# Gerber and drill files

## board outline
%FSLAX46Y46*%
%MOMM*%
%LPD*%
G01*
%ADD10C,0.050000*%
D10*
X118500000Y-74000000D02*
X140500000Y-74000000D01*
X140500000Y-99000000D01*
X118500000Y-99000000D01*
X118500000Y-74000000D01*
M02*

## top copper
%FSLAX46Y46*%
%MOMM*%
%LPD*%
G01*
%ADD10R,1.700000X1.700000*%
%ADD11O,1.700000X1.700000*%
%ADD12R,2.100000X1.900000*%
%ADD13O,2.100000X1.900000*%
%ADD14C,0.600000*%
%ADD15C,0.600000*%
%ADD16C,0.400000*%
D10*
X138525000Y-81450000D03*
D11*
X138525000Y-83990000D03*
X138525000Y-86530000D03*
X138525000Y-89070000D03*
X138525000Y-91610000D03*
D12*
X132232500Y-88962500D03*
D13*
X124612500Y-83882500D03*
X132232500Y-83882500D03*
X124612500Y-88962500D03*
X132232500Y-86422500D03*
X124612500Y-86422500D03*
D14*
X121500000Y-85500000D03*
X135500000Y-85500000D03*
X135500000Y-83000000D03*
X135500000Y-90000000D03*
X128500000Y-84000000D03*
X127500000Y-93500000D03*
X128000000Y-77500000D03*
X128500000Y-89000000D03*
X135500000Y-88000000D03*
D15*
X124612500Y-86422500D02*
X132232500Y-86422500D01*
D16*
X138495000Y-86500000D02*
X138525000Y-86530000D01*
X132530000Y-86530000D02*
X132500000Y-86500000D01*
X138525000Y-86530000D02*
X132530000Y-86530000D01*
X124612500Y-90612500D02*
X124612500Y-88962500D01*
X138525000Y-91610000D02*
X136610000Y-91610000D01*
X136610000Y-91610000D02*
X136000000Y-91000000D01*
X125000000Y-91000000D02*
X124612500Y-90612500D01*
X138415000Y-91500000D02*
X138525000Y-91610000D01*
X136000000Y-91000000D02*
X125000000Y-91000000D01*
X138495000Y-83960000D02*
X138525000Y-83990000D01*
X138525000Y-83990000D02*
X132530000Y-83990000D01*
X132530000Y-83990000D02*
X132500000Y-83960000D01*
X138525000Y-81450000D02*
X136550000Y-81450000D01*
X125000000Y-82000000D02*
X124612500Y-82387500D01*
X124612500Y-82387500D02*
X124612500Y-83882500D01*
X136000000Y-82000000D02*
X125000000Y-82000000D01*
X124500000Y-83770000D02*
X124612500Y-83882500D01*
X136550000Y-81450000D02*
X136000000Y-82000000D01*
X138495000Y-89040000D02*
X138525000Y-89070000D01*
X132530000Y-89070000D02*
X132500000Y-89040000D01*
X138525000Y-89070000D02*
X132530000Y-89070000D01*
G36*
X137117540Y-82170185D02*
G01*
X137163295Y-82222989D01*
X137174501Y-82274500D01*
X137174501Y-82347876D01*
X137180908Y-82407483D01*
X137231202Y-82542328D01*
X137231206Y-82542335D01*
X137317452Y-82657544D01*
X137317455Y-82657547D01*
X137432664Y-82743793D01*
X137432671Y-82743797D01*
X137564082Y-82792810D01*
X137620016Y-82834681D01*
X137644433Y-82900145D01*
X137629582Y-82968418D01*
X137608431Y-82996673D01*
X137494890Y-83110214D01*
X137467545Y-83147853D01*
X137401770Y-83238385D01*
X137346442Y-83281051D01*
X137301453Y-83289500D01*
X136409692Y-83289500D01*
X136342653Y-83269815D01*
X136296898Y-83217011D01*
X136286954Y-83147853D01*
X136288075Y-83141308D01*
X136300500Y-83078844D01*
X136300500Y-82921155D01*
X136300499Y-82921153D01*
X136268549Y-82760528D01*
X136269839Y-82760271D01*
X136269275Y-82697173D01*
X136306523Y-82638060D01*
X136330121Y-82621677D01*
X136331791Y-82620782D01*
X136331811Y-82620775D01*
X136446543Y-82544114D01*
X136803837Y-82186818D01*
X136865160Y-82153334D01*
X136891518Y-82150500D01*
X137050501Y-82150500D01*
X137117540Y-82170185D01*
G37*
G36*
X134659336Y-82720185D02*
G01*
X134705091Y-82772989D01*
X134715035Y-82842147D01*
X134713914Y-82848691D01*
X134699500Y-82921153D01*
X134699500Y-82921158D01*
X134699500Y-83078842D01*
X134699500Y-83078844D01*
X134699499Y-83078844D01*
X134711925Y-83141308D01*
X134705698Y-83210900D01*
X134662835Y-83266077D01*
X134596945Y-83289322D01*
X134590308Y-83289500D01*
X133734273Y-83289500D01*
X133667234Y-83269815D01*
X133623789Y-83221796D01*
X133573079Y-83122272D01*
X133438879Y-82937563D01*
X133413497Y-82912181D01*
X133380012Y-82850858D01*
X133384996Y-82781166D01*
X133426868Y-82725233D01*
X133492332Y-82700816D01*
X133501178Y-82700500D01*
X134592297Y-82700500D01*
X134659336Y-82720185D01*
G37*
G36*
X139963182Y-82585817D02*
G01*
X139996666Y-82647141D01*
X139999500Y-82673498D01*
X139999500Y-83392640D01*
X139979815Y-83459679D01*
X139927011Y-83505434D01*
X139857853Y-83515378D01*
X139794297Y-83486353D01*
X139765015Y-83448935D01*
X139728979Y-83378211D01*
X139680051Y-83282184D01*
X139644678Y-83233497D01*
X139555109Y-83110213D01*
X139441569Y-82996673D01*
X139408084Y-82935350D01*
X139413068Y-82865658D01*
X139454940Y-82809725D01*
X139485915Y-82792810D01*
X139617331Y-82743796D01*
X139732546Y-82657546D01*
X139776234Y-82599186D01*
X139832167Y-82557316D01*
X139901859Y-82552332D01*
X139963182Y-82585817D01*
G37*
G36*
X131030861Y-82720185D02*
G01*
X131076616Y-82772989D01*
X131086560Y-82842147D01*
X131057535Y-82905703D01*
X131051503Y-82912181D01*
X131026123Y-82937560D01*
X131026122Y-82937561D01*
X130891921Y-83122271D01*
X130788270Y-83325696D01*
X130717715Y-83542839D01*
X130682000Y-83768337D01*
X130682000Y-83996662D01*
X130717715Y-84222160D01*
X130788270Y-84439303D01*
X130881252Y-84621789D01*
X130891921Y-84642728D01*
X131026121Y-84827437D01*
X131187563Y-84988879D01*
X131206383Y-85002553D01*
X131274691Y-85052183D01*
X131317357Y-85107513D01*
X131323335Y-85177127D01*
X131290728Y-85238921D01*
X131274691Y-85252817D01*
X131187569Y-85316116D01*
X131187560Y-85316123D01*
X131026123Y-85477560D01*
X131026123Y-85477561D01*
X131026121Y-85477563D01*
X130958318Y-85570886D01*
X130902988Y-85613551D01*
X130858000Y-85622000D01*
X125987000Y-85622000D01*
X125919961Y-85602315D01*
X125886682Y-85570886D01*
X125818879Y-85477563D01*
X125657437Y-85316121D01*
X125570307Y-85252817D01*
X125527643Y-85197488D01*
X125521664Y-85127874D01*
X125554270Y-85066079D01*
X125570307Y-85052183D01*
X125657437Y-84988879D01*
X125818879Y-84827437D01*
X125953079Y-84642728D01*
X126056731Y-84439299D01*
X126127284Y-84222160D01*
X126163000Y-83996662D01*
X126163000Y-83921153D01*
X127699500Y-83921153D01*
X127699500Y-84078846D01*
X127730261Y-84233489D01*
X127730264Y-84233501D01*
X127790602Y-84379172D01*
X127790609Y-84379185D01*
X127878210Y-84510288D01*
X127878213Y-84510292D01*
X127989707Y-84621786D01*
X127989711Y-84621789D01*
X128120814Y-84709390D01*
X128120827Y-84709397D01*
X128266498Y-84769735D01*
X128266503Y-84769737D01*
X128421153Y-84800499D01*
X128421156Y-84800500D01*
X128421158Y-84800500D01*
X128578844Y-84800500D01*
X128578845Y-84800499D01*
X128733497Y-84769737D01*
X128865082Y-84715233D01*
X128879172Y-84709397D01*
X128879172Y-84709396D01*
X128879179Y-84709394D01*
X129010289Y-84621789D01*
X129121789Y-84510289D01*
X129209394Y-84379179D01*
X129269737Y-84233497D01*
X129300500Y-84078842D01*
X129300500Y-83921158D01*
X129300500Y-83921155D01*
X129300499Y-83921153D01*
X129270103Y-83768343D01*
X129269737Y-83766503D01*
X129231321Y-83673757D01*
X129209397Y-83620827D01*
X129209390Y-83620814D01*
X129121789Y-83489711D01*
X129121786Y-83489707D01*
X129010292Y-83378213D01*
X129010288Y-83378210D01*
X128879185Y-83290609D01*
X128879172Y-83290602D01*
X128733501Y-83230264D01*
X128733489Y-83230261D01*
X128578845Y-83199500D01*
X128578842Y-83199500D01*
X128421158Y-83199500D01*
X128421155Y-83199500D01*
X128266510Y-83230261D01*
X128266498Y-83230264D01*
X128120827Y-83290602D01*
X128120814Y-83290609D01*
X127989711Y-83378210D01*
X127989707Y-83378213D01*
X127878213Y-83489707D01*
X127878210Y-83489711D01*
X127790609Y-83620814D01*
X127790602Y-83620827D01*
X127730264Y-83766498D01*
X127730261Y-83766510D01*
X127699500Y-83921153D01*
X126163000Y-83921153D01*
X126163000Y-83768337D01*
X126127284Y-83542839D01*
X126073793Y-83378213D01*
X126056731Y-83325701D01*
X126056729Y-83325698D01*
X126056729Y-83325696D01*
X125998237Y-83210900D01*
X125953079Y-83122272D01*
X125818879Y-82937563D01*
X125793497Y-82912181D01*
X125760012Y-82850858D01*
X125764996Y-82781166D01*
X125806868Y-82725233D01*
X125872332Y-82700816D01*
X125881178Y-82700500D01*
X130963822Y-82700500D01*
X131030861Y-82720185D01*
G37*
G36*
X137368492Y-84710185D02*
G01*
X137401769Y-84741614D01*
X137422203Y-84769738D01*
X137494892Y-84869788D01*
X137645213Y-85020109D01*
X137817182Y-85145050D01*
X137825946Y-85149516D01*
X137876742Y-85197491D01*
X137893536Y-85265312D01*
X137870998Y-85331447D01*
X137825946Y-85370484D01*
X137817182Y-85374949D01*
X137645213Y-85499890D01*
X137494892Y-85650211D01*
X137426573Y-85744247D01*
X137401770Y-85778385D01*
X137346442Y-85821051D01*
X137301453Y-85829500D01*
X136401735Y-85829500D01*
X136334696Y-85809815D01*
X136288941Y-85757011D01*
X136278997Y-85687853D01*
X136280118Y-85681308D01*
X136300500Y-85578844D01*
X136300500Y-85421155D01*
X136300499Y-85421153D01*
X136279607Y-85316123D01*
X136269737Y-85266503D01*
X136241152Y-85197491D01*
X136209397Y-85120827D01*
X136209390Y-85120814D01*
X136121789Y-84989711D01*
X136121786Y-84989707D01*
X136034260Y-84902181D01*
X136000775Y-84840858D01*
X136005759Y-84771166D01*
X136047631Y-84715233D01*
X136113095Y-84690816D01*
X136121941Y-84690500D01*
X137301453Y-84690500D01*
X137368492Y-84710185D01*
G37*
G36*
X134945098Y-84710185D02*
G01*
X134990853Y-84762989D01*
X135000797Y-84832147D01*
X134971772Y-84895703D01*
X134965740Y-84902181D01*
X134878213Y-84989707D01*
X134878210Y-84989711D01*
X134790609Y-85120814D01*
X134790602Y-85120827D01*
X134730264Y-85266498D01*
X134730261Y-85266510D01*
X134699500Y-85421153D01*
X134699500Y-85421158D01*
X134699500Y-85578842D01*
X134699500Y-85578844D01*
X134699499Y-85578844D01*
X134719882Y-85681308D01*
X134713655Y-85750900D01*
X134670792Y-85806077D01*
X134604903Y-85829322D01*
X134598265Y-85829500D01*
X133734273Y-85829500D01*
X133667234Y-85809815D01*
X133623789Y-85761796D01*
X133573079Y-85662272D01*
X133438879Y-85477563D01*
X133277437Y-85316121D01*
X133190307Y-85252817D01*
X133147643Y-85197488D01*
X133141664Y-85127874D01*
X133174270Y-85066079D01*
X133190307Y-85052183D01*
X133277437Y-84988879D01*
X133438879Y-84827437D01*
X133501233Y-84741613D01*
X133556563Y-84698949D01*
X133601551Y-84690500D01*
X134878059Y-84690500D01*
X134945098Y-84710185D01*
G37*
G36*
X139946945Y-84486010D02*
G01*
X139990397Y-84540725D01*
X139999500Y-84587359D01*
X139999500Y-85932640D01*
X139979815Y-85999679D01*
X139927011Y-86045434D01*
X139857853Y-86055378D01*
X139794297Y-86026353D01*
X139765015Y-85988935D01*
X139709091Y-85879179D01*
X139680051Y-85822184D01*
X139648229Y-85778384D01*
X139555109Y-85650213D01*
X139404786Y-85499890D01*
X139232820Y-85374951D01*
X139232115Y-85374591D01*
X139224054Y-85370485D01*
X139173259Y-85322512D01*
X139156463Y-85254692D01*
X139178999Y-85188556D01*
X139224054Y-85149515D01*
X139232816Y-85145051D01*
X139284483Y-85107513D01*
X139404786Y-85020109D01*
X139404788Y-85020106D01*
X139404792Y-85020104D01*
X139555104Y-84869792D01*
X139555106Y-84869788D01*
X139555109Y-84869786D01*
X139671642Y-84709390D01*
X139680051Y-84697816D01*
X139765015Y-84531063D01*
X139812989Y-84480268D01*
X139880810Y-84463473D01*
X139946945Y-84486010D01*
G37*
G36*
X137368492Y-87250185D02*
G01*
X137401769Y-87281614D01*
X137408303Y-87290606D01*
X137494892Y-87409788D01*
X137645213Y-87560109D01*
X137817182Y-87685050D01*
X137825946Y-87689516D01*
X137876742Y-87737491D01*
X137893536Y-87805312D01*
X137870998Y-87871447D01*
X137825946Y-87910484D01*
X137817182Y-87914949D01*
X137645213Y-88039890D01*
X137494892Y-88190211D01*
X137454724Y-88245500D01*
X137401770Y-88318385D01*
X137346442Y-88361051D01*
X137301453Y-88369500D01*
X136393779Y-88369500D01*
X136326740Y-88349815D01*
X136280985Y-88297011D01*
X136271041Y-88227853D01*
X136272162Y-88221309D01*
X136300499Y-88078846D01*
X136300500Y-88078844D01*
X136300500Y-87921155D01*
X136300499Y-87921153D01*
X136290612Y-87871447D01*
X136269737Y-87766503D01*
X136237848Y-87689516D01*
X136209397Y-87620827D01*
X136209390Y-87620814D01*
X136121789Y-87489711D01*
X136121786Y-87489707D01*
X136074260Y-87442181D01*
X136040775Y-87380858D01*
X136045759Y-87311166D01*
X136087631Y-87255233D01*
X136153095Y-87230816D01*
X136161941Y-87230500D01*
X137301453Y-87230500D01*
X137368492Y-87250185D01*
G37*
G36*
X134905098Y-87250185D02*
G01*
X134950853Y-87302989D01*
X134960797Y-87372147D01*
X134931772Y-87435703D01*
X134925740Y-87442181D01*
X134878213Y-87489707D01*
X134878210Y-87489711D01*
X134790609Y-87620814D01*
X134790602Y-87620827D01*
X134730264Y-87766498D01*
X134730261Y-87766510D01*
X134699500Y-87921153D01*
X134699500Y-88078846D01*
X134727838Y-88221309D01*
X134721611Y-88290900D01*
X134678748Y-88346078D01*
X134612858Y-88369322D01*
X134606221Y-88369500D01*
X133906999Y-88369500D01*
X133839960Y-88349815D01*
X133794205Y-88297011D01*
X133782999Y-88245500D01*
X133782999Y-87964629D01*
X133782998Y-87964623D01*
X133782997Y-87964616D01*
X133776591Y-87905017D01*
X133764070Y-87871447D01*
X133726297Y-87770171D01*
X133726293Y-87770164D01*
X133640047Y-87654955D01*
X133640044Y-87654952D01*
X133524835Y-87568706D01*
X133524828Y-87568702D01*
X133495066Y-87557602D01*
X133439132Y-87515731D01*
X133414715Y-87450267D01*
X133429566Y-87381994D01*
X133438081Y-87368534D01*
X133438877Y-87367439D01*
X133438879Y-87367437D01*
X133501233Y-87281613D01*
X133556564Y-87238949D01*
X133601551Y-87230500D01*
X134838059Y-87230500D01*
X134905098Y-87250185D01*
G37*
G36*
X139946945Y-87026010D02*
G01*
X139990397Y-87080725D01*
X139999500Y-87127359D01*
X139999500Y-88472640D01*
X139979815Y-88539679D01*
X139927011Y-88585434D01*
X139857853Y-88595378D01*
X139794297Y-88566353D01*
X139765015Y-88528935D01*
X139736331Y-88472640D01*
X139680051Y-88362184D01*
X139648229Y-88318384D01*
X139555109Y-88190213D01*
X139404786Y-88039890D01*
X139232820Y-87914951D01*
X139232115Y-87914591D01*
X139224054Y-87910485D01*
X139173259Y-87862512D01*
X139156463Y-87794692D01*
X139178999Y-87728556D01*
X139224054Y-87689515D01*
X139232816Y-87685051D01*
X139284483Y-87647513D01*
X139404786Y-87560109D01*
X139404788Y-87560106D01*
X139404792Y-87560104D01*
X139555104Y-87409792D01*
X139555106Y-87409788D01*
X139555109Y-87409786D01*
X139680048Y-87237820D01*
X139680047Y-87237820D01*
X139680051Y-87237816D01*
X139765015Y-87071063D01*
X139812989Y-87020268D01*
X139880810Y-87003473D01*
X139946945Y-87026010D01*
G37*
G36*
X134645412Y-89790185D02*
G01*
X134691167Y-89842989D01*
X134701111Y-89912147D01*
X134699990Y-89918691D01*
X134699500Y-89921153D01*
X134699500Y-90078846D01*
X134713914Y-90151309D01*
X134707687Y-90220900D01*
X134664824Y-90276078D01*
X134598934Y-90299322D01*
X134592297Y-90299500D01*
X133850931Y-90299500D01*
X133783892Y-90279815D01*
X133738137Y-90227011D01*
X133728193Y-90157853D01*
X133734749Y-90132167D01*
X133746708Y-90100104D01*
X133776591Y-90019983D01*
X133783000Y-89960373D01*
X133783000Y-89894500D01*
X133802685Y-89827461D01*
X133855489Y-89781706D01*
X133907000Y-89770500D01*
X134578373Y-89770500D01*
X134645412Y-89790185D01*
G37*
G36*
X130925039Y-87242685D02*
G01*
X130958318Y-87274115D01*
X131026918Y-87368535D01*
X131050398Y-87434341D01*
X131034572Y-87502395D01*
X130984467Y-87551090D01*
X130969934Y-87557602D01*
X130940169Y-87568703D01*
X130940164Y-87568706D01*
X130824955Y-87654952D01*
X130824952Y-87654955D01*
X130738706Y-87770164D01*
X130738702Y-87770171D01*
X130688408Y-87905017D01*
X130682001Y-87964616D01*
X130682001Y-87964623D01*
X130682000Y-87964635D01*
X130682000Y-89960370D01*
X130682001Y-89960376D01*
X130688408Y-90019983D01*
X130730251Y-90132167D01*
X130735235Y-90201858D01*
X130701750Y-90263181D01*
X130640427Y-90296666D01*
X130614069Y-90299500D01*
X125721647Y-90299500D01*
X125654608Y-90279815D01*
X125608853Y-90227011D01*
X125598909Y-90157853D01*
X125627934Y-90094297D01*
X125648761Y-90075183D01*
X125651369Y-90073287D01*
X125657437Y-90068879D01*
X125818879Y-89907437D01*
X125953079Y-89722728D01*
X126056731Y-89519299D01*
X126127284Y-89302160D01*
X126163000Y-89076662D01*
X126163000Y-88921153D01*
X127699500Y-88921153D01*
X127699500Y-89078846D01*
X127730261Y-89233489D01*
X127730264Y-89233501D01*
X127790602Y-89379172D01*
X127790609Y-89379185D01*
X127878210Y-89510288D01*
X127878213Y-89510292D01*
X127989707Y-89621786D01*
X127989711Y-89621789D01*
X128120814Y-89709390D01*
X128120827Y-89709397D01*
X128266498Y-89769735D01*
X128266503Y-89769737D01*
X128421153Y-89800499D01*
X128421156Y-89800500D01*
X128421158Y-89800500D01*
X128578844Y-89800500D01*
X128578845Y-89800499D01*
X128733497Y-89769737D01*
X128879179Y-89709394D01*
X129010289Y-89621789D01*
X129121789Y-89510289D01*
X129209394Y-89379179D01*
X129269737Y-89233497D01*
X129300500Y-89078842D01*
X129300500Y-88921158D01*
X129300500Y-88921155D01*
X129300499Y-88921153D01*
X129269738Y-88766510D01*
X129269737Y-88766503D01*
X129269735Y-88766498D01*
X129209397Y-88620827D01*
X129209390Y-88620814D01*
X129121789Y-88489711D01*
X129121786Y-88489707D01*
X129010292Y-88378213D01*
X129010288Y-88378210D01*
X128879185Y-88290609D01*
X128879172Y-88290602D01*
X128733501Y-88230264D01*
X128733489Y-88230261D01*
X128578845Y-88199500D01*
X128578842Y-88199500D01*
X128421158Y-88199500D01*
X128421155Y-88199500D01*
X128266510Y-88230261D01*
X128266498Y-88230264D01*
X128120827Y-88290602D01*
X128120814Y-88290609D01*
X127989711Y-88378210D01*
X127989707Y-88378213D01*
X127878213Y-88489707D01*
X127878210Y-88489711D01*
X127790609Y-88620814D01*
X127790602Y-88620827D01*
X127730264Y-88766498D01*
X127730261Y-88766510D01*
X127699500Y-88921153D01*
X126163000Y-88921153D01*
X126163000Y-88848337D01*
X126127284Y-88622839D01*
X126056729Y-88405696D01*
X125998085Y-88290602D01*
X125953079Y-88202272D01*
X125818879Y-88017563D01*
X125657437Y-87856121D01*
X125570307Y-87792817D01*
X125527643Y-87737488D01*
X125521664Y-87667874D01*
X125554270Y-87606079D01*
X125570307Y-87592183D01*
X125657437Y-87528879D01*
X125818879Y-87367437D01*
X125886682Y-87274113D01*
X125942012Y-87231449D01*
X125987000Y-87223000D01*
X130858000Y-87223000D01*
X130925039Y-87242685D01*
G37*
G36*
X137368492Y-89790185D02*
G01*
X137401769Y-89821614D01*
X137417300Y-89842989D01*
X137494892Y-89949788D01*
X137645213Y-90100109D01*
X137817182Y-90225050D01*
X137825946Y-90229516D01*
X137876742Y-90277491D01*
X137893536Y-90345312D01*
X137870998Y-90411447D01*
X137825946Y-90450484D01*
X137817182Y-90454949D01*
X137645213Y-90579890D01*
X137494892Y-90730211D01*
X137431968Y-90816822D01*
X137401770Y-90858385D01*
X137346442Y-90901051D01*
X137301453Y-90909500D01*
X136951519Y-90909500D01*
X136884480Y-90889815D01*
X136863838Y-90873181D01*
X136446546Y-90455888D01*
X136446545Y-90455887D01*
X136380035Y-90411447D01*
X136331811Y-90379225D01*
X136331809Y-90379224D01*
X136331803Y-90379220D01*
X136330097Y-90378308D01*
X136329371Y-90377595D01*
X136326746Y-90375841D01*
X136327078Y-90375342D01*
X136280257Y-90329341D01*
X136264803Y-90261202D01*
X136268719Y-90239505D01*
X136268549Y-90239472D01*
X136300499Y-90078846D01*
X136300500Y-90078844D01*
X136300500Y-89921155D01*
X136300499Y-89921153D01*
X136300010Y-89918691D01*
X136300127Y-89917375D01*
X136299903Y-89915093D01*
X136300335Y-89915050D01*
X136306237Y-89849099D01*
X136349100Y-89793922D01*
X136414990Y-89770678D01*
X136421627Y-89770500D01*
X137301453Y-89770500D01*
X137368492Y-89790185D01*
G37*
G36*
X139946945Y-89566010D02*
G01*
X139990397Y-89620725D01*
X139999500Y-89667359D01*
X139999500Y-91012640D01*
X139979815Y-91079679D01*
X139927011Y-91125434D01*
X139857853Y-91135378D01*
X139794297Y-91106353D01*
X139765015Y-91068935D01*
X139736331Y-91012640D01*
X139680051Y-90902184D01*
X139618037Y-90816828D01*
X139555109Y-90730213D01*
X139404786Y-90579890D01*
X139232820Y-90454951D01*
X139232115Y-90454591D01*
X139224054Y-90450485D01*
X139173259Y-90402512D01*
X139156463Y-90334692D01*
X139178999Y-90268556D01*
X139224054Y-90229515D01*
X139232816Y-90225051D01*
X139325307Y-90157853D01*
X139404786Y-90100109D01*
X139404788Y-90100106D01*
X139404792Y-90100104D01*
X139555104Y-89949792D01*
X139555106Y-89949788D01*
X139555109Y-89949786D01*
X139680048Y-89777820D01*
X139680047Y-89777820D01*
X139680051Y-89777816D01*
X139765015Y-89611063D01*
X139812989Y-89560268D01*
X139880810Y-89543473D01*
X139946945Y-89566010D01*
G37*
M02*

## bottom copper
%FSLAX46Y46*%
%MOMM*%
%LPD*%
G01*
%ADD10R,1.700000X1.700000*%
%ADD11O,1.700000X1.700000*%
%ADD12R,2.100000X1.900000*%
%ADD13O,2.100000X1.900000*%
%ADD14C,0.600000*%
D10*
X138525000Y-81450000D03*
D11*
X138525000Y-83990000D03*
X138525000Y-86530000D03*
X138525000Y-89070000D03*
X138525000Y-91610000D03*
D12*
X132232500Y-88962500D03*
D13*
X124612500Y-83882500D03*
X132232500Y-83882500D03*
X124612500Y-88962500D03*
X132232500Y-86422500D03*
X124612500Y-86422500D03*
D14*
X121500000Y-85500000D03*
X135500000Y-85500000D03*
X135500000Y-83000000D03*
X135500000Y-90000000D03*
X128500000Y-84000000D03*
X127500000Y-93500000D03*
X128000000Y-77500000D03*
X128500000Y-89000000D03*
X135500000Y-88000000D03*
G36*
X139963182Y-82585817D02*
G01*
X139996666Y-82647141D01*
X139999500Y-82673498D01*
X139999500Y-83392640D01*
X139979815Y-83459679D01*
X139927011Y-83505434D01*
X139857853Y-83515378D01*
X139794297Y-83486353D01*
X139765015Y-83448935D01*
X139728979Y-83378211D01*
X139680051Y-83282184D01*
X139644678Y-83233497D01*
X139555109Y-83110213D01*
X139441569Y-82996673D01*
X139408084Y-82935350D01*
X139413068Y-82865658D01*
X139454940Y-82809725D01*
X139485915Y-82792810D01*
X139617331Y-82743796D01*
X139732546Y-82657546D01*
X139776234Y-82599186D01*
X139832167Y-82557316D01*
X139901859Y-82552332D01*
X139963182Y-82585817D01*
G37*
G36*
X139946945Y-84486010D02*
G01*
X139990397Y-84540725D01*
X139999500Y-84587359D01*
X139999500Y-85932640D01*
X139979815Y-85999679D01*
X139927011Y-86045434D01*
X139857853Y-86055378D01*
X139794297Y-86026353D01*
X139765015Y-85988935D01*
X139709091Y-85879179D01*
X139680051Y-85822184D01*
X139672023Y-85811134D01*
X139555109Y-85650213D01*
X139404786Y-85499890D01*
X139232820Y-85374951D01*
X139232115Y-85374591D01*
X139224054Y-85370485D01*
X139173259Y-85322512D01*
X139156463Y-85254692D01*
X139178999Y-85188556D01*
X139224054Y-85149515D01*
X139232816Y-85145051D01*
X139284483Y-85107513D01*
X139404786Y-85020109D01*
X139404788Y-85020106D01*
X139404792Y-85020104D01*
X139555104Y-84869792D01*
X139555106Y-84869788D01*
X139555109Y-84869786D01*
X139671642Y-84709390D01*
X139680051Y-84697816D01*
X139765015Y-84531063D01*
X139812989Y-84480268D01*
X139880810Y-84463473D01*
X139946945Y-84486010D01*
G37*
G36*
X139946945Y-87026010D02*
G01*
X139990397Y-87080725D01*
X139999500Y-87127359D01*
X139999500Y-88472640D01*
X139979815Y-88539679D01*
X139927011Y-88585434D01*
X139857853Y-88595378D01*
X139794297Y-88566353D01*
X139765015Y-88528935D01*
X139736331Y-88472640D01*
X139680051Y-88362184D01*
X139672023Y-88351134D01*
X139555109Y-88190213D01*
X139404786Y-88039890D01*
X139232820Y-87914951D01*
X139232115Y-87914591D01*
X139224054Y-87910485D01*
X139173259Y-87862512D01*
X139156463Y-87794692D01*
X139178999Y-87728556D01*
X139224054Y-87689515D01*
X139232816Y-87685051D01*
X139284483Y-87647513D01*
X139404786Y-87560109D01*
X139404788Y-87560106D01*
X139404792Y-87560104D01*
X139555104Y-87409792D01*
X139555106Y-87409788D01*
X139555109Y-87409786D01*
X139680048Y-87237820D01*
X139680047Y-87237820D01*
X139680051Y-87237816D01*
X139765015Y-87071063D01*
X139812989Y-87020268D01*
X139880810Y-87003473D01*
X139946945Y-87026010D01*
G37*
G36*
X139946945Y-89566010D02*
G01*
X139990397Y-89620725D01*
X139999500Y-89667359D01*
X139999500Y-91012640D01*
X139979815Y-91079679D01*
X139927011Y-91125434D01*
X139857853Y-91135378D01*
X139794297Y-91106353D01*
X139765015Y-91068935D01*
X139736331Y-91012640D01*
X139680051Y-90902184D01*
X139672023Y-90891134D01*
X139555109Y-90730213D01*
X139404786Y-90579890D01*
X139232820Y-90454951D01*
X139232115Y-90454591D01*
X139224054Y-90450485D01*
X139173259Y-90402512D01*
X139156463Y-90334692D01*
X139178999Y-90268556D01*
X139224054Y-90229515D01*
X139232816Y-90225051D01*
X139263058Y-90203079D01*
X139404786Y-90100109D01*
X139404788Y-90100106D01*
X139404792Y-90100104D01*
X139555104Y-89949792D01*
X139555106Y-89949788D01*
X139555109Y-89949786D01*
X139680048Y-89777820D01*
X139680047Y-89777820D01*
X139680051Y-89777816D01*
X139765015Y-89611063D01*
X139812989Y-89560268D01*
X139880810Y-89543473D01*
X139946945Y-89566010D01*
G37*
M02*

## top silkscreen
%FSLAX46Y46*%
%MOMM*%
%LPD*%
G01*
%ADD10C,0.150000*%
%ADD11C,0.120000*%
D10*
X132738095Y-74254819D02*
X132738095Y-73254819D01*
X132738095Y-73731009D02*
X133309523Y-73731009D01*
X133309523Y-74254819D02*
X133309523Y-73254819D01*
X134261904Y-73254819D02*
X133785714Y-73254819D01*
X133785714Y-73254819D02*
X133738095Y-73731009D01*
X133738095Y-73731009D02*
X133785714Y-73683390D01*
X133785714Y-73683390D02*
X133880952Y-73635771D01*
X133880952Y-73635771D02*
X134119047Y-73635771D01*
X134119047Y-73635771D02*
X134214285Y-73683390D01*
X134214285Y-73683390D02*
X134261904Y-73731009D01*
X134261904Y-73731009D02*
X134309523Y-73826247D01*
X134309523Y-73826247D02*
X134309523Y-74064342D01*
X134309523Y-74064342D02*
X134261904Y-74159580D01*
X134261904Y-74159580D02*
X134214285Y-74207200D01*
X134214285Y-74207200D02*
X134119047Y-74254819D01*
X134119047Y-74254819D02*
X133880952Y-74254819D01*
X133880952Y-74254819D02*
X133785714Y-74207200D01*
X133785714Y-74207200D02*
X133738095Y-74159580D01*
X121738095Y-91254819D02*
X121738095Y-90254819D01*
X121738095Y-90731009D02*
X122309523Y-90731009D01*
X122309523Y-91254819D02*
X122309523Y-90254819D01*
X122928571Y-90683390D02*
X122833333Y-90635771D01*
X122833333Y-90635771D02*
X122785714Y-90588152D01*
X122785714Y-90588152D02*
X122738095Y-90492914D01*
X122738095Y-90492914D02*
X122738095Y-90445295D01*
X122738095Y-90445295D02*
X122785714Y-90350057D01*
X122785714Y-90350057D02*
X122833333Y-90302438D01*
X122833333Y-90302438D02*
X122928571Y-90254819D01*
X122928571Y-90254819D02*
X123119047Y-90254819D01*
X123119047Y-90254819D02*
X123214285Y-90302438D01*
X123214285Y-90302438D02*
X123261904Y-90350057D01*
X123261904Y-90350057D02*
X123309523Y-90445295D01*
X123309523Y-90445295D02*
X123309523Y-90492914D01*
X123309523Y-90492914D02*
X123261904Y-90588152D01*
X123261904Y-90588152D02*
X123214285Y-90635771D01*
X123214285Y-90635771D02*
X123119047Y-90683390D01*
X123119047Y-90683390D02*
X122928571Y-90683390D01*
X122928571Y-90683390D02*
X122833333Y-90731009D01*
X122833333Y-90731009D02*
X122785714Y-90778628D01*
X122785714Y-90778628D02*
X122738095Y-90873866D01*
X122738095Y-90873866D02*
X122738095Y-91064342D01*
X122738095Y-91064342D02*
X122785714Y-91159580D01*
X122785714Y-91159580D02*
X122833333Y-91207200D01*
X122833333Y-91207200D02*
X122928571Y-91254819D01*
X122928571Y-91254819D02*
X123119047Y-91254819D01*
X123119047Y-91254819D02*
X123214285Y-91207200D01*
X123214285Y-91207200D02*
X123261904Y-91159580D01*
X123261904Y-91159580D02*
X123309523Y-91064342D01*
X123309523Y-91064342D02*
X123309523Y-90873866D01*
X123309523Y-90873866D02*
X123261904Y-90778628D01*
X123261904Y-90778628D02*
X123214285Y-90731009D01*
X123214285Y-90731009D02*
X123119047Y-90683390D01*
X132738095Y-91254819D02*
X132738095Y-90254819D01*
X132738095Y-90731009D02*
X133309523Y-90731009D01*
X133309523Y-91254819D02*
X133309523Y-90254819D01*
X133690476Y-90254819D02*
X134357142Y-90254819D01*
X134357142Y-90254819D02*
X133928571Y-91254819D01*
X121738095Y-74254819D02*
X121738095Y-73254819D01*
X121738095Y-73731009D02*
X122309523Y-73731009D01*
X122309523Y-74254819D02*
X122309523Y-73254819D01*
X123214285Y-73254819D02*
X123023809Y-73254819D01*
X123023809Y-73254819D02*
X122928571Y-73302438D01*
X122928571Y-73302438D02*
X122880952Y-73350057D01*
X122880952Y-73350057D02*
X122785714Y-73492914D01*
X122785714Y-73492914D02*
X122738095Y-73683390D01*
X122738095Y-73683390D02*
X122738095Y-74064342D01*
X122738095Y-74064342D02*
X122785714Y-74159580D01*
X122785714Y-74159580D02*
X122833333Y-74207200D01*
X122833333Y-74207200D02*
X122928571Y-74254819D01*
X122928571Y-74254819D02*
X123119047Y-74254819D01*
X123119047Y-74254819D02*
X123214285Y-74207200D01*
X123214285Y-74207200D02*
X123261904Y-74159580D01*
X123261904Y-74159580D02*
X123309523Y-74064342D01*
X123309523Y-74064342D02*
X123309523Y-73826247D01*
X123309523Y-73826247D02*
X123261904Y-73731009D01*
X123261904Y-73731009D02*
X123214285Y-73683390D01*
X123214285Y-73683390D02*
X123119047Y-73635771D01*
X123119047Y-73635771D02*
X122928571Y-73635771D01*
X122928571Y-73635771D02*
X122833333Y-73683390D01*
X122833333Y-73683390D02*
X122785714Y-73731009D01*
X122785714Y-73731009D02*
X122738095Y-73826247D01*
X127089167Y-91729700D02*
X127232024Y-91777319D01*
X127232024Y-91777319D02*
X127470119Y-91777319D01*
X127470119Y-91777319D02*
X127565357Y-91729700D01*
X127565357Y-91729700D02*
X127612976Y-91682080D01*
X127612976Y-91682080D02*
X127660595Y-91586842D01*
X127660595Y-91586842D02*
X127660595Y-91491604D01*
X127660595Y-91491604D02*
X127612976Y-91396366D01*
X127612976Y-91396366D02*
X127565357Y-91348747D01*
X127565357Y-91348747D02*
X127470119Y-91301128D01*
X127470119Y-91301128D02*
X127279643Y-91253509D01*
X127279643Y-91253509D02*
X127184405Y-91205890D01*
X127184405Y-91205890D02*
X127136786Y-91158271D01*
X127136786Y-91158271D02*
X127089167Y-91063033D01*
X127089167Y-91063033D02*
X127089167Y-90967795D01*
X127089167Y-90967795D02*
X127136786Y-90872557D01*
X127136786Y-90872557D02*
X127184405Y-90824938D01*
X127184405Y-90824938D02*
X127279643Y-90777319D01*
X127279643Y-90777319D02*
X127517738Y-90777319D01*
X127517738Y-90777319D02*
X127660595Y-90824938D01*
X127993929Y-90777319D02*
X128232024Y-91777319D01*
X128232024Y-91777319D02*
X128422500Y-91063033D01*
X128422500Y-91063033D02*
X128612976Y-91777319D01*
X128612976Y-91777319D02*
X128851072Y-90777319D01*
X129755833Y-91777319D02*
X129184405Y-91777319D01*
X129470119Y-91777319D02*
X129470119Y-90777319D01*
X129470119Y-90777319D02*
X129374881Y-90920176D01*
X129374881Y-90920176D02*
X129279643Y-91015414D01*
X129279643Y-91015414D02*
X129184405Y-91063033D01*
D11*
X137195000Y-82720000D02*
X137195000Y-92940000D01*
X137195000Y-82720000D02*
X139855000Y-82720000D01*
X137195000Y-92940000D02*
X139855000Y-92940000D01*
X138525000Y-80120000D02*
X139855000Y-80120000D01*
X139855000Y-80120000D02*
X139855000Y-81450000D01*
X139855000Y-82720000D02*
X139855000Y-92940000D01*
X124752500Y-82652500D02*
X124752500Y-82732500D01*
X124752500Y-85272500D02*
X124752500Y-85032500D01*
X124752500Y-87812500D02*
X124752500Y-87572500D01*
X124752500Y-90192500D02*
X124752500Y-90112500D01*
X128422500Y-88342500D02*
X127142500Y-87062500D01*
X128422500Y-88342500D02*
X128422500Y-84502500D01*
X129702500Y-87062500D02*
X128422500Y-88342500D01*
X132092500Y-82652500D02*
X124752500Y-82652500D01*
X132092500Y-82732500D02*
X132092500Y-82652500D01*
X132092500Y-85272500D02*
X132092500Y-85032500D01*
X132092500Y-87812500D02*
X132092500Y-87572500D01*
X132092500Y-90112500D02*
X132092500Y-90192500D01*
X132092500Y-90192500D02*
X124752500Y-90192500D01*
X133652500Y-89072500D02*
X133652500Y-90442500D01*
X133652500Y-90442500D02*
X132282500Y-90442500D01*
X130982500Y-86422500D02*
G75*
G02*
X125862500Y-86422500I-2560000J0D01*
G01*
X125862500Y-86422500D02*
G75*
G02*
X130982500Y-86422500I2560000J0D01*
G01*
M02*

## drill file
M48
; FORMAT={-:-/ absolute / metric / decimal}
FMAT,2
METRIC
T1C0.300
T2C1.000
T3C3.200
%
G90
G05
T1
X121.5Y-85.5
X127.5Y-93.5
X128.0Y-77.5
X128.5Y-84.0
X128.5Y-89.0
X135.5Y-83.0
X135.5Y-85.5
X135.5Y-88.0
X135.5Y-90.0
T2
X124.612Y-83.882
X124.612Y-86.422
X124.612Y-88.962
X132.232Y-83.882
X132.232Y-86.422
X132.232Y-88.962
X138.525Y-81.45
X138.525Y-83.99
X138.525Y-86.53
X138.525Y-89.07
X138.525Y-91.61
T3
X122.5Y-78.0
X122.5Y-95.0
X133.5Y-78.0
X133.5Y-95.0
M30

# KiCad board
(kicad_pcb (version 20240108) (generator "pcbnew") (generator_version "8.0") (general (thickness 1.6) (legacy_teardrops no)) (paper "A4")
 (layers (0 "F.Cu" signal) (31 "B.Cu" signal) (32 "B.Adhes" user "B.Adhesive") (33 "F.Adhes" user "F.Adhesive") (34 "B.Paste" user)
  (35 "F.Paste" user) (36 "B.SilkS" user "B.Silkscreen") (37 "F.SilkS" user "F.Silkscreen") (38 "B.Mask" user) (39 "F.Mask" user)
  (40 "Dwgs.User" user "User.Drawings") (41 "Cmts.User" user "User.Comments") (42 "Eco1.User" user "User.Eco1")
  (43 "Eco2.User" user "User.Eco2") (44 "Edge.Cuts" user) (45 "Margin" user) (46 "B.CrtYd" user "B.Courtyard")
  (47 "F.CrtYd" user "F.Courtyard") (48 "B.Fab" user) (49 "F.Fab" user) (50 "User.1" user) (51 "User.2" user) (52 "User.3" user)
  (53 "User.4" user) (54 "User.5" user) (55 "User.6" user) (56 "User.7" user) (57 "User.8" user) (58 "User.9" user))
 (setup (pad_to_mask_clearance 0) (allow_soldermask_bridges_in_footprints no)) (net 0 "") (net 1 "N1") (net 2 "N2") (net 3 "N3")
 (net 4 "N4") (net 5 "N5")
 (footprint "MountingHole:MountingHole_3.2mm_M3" (layer "F.Cu") (at 133.5 78)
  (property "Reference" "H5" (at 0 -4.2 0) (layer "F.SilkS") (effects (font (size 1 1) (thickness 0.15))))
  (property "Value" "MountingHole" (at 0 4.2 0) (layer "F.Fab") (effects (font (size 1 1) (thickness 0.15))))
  (pad "" np_thru_hole circle (at 0 0) (size 3.2 3.2) (drill 3.2) (layers "*.Cu" "*.Mask")))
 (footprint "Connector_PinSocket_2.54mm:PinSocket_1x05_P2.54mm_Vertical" (layer "F.Cu") (at 138.525 81.45)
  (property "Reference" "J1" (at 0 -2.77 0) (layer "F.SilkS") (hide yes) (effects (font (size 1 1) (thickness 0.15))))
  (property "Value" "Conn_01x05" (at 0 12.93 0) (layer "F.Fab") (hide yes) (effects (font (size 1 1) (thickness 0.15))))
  (fp_line (start -1.33 1.27) (end -1.33 11.49) (stroke (width 0.12) (type solid)) (layer "F.SilkS"))
  (fp_line (start -1.33 1.27) (end 1.33 1.27) (stroke (width 0.12) (type solid)) (layer "F.SilkS"))
  (fp_line (start -1.33 11.49) (end 1.33 11.49) (stroke (width 0.12) (type solid)) (layer "F.SilkS"))
  (fp_line (start 0 -1.33) (end 1.33 -1.33) (stroke (width 0.12) (type solid)) (layer "F.SilkS"))
  (fp_line (start 1.33 -1.33) (end 1.33 0) (stroke (width 0.12) (type solid)) (layer "F.SilkS"))
  (fp_line (start 1.33 1.27) (end 1.33 11.49) (stroke (width 0.12) (type solid)) (layer "F.SilkS"))
  (pad "1" thru_hole rect (at 0 0) (size 1.7 1.7) (drill 1) (layers "*.Cu" "*.Mask") (remove_unused_layers no) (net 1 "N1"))
  (pad "2" thru_hole oval (at 0 2.54) (size 1.7 1.7) (drill 1) (layers "*.Cu" "*.Mask") (remove_unused_layers no) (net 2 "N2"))
  (pad "3" thru_hole oval (at 0 5.08) (size 1.7 1.7) (drill 1) (layers "*.Cu" "*.Mask") (remove_unused_layers no) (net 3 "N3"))
  (pad "4" thru_hole oval (at 0 7.62) (size 1.7 1.7) (drill 1) (layers "*.Cu" "*.Mask") (remove_unused_layers no) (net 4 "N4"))
  (pad "5" thru_hole oval (at 0 10.16) (size 1.7 1.7) (drill 1) (layers "*.Cu" "*.Mask") (remove_unused_layers no) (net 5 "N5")))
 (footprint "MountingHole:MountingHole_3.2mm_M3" (layer "F.Cu") (at 122.5 95)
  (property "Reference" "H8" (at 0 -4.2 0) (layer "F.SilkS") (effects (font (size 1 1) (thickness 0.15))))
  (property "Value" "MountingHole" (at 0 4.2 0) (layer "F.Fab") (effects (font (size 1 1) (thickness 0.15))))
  (pad "" np_thru_hole circle (at 0 0) (size 3.2 3.2) (drill 3.2) (layers "*.Cu" "*.Mask")))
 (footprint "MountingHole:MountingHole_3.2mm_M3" (layer "F.Cu") (at 133.5 95)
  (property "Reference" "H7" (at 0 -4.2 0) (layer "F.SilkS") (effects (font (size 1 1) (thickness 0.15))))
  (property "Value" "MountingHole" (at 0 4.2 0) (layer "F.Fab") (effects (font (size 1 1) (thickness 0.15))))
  (pad "" np_thru_hole circle (at 0 0) (size 3.2 3.2) (drill 3.2) (layers "*.Cu" "*.Mask")))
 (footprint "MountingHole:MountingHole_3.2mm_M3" (layer "F.Cu") (at 122.5 78)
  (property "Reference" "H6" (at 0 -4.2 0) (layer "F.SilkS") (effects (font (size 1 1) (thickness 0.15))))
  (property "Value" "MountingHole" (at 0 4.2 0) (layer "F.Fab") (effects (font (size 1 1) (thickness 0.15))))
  (pad "" np_thru_hole circle (at 0 0) (size 3.2 3.2) (drill 3.2) (layers "*.Cu" "*.Mask")))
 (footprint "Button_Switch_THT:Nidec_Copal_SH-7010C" (layer "F.Cu") (at 132.2325 88.9625 180)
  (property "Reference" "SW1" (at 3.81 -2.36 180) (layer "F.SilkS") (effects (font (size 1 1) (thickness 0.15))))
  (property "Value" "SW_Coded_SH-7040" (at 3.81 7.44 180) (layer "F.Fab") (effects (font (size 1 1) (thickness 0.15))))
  (fp_line (start 7.48 6.31) (end 7.48 6.23) (stroke (width 0.12) (type solid)) (layer "F.SilkS"))
  (fp_line (start 7.48 3.69) (end 7.48 3.93) (stroke (width 0.12) (type solid)) (layer "F.SilkS"))
  (fp_line (start 7.48 1.15) (end 7.48 1.39) (stroke (width 0.12) (type solid)) (layer "F.SilkS"))
  (fp_line (start 7.48 -1.23) (end 7.48 -1.15) (stroke (width 0.12) (type solid)) (layer "F.SilkS"))
  (fp_line (start 3.81 0.62) (end 5.09 1.9) (stroke (width 0.12) (type solid)) (layer "F.SilkS"))
  (fp_line (start 3.81 0.62) (end 3.81 4.46) (stroke (width 0.12) (type solid)) (layer "F.SilkS"))
  (fp_line (start 2.53 1.9) (end 3.81 0.62) (stroke (width 0.12) (type solid)) (layer "F.SilkS"))
  (fp_line (start 0.14 6.31) (end 7.48 6.31) (stroke (width 0.12) (type solid)) (layer "F.SilkS"))
  (fp_line (start 0.14 6.23) (end 0.14 6.31) (stroke (width 0.12) (type solid)) (layer "F.SilkS"))
  (fp_line (start 0.14 3.69) (end 0.14 3.93) (stroke (width 0.12) (type solid)) (layer "F.SilkS"))
  (fp_line (start 0.14 1.15) (end 0.14 1.39) (stroke (width 0.12) (type solid)) (layer "F.SilkS"))
  (fp_line (start 0.14 -1.15) (end 0.14 -1.23) (stroke (width 0.12) (type solid)) (layer "F.SilkS"))
  (fp_line (start 0.14 -1.23) (end 7.48 -1.23) (stroke (width 0.12) (type solid)) (layer "F.SilkS"))
  (fp_line (start -1.42 -0.11) (end -1.42 -1.48) (stroke (width 0.12) (type solid)) (layer "F.SilkS"))
  (fp_line (start -1.42 -1.48) (end -0.05 -1.48) (stroke (width 0.12) (type solid)) (layer "F.SilkS"))
  (fp_circle (center 3.81 2.54) (end 6.37 2.54) (stroke (width 0.12) (type solid)) (fill none) (layer "F.SilkS"))
  (pad "1" thru_hole rect (at 0 0 180) (size 2.1 1.9) (drill 1) (layers "*.Cu" "*.Mask") (remove_unused_layers no) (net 4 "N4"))
  (pad "2" thru_hole oval (at 7.62 5.08 180) (size 2.1 1.9) (drill 1) (layers "*.Cu" "*.Mask") (remove_unused_layers no) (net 1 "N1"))
  (pad "4" thru_hole oval (at 0 5.08 180) (size 2.1 1.9) (drill 1) (layers "*.Cu" "*.Mask") (remove_unused_layers no) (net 2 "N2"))
  (pad "8" thru_hole oval (at 7.62 0 180) (size 2.1 1.9) (drill 1) (layers "*.Cu" "*.Mask") (remove_unused_layers no) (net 5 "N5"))
  (pad "C" thru_hole oval (at 0 2.54 180) (size 2.1 1.9) (drill 1) (layers "*.Cu" "*.Mask") (remove_unused_layers no) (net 3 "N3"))
  (pad "C" thru_hole oval (at 7.62 2.54 180) (size 2.1 1.9) (drill 1) (layers "*.Cu" "*.Mask") (remove_unused_layers no) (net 3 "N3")))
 (gr_rect (start 118.5 74) (end 140.5 99) (stroke (width 0.05) (type default)) (fill none) (layer "Edge.Cuts"))
 (via (at 121.5 85.5) (size 0.6) (drill 0.3) (layers "F.Cu" "B.Cu") (free yes) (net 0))
 (via (at 135.5 85.5) (size 0.6) (drill 0.3) (layers "F.Cu" "B.Cu") (free yes) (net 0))
 (via (at 135.5 83) (size 0.6) (drill 0.3) (layers "F.Cu" "B.Cu") (free yes) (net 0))
 (via (at 135.5 90) (size 0.6) (drill 0.3) (layers "F.Cu" "B.Cu") (free yes) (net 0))
 (via (at 128.5 84) (size 0.6) (drill 0.3) (layers "F.Cu" "B.Cu") (free yes) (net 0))
 (via (at 127.5 93.5) (size 0.6) (drill 0.3) (layers "F.Cu" "B.Cu") (free yes) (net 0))
 (via (at 128 77.5) (size 0.6) (drill 0.3) (layers "F.Cu" "B.Cu") (free yes) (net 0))
 (via (at 128.5 89) (size 0.6) (drill 0.3) (layers "F.Cu" "B.Cu") (free yes) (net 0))
 (via (at 135.5 88) (size 0.6) (drill 0.3) (layers "F.Cu" "B.Cu") (free yes) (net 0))
 (segment (start 124.6125 86.4225) (end 132.2325 86.4225) (width 0.6) (layer "F.Cu") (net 3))
 (segment (start 138.495 86.5) (end 138.525 86.53) (width 0.4) (layer "F.Cu") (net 3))
 (segment (start 132.53 86.53) (end 132.5 86.5) (width 0.4) (layer "F.Cu") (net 3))
 (segment (start 138.525 86.53) (end 132.53 86.53) (width 0.4) (layer "F.Cu") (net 3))
 (segment (start 124.6125 90.6125) (end 124.6125 88.9625) (width 0.4) (layer "F.Cu") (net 5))
 (segment (start 138.525 91.61) (end 136.61 91.61) (width 0.4) (layer "F.Cu") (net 5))
 (segment (start 136.61 91.61) (end 136 91) (width 0.4) (layer "F.Cu") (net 5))
 (segment (start 125 91) (end 124.6125 90.6125) (width 0.4) (layer "F.Cu") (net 5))
 (segment (start 138.415 91.5) (end 138.525 91.61) (width 0.4) (layer "F.Cu") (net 5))
 (segment (start 136 91) (end 125 91) (width 0.4) (layer "F.Cu") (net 5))
 (segment (start 138.495 83.96) (end 138.525 83.99) (width 0.4) (layer "F.Cu") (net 2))
 (segment (start 138.525 83.99) (end 132.53 83.99) (width 0.4) (layer "F.Cu") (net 2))
 (segment (start 132.53 83.99) (end 132.5 83.96) (width 0.4) (layer "F.Cu") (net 2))
 (segment (start 138.525 81.45) (end 136.55 81.45) (width 0.4) (layer "F.Cu") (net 1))
 (segment (start 125 82) (end 124.6125 82.3875) (width 0.4) (layer "F.Cu") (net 1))
 (segment (start 124.6125 82.3875) (end 124.6125 83.8825) (width 0.4) (layer "F.Cu") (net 1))
 (segment (start 136 82) (end 125 82) (width 0.4) (layer "F.Cu") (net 1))
 (segment (start 124.5 83.77) (end 124.6125 83.8825) (width 0.4) (layer "F.Cu") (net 1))
 (segment (start 136.55 81.45) (end 136 82) (width 0.4) (layer "F.Cu") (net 1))
 (segment (start 138.495 89.04) (end 138.525 89.07) (width 0.4) (layer "F.Cu") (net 4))
 (segment (start 132.53 89.07) (end 132.5 89.04) (width 0.4) (layer "F.Cu") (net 4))
 (segment (start 138.525 89.07) (end 132.53 89.07) (width 0.4) (layer "F.Cu") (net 4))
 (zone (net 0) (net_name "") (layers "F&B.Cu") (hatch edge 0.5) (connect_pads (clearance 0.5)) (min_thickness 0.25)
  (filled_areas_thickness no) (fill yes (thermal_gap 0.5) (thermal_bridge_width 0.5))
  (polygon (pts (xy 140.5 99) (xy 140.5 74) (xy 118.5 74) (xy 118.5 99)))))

